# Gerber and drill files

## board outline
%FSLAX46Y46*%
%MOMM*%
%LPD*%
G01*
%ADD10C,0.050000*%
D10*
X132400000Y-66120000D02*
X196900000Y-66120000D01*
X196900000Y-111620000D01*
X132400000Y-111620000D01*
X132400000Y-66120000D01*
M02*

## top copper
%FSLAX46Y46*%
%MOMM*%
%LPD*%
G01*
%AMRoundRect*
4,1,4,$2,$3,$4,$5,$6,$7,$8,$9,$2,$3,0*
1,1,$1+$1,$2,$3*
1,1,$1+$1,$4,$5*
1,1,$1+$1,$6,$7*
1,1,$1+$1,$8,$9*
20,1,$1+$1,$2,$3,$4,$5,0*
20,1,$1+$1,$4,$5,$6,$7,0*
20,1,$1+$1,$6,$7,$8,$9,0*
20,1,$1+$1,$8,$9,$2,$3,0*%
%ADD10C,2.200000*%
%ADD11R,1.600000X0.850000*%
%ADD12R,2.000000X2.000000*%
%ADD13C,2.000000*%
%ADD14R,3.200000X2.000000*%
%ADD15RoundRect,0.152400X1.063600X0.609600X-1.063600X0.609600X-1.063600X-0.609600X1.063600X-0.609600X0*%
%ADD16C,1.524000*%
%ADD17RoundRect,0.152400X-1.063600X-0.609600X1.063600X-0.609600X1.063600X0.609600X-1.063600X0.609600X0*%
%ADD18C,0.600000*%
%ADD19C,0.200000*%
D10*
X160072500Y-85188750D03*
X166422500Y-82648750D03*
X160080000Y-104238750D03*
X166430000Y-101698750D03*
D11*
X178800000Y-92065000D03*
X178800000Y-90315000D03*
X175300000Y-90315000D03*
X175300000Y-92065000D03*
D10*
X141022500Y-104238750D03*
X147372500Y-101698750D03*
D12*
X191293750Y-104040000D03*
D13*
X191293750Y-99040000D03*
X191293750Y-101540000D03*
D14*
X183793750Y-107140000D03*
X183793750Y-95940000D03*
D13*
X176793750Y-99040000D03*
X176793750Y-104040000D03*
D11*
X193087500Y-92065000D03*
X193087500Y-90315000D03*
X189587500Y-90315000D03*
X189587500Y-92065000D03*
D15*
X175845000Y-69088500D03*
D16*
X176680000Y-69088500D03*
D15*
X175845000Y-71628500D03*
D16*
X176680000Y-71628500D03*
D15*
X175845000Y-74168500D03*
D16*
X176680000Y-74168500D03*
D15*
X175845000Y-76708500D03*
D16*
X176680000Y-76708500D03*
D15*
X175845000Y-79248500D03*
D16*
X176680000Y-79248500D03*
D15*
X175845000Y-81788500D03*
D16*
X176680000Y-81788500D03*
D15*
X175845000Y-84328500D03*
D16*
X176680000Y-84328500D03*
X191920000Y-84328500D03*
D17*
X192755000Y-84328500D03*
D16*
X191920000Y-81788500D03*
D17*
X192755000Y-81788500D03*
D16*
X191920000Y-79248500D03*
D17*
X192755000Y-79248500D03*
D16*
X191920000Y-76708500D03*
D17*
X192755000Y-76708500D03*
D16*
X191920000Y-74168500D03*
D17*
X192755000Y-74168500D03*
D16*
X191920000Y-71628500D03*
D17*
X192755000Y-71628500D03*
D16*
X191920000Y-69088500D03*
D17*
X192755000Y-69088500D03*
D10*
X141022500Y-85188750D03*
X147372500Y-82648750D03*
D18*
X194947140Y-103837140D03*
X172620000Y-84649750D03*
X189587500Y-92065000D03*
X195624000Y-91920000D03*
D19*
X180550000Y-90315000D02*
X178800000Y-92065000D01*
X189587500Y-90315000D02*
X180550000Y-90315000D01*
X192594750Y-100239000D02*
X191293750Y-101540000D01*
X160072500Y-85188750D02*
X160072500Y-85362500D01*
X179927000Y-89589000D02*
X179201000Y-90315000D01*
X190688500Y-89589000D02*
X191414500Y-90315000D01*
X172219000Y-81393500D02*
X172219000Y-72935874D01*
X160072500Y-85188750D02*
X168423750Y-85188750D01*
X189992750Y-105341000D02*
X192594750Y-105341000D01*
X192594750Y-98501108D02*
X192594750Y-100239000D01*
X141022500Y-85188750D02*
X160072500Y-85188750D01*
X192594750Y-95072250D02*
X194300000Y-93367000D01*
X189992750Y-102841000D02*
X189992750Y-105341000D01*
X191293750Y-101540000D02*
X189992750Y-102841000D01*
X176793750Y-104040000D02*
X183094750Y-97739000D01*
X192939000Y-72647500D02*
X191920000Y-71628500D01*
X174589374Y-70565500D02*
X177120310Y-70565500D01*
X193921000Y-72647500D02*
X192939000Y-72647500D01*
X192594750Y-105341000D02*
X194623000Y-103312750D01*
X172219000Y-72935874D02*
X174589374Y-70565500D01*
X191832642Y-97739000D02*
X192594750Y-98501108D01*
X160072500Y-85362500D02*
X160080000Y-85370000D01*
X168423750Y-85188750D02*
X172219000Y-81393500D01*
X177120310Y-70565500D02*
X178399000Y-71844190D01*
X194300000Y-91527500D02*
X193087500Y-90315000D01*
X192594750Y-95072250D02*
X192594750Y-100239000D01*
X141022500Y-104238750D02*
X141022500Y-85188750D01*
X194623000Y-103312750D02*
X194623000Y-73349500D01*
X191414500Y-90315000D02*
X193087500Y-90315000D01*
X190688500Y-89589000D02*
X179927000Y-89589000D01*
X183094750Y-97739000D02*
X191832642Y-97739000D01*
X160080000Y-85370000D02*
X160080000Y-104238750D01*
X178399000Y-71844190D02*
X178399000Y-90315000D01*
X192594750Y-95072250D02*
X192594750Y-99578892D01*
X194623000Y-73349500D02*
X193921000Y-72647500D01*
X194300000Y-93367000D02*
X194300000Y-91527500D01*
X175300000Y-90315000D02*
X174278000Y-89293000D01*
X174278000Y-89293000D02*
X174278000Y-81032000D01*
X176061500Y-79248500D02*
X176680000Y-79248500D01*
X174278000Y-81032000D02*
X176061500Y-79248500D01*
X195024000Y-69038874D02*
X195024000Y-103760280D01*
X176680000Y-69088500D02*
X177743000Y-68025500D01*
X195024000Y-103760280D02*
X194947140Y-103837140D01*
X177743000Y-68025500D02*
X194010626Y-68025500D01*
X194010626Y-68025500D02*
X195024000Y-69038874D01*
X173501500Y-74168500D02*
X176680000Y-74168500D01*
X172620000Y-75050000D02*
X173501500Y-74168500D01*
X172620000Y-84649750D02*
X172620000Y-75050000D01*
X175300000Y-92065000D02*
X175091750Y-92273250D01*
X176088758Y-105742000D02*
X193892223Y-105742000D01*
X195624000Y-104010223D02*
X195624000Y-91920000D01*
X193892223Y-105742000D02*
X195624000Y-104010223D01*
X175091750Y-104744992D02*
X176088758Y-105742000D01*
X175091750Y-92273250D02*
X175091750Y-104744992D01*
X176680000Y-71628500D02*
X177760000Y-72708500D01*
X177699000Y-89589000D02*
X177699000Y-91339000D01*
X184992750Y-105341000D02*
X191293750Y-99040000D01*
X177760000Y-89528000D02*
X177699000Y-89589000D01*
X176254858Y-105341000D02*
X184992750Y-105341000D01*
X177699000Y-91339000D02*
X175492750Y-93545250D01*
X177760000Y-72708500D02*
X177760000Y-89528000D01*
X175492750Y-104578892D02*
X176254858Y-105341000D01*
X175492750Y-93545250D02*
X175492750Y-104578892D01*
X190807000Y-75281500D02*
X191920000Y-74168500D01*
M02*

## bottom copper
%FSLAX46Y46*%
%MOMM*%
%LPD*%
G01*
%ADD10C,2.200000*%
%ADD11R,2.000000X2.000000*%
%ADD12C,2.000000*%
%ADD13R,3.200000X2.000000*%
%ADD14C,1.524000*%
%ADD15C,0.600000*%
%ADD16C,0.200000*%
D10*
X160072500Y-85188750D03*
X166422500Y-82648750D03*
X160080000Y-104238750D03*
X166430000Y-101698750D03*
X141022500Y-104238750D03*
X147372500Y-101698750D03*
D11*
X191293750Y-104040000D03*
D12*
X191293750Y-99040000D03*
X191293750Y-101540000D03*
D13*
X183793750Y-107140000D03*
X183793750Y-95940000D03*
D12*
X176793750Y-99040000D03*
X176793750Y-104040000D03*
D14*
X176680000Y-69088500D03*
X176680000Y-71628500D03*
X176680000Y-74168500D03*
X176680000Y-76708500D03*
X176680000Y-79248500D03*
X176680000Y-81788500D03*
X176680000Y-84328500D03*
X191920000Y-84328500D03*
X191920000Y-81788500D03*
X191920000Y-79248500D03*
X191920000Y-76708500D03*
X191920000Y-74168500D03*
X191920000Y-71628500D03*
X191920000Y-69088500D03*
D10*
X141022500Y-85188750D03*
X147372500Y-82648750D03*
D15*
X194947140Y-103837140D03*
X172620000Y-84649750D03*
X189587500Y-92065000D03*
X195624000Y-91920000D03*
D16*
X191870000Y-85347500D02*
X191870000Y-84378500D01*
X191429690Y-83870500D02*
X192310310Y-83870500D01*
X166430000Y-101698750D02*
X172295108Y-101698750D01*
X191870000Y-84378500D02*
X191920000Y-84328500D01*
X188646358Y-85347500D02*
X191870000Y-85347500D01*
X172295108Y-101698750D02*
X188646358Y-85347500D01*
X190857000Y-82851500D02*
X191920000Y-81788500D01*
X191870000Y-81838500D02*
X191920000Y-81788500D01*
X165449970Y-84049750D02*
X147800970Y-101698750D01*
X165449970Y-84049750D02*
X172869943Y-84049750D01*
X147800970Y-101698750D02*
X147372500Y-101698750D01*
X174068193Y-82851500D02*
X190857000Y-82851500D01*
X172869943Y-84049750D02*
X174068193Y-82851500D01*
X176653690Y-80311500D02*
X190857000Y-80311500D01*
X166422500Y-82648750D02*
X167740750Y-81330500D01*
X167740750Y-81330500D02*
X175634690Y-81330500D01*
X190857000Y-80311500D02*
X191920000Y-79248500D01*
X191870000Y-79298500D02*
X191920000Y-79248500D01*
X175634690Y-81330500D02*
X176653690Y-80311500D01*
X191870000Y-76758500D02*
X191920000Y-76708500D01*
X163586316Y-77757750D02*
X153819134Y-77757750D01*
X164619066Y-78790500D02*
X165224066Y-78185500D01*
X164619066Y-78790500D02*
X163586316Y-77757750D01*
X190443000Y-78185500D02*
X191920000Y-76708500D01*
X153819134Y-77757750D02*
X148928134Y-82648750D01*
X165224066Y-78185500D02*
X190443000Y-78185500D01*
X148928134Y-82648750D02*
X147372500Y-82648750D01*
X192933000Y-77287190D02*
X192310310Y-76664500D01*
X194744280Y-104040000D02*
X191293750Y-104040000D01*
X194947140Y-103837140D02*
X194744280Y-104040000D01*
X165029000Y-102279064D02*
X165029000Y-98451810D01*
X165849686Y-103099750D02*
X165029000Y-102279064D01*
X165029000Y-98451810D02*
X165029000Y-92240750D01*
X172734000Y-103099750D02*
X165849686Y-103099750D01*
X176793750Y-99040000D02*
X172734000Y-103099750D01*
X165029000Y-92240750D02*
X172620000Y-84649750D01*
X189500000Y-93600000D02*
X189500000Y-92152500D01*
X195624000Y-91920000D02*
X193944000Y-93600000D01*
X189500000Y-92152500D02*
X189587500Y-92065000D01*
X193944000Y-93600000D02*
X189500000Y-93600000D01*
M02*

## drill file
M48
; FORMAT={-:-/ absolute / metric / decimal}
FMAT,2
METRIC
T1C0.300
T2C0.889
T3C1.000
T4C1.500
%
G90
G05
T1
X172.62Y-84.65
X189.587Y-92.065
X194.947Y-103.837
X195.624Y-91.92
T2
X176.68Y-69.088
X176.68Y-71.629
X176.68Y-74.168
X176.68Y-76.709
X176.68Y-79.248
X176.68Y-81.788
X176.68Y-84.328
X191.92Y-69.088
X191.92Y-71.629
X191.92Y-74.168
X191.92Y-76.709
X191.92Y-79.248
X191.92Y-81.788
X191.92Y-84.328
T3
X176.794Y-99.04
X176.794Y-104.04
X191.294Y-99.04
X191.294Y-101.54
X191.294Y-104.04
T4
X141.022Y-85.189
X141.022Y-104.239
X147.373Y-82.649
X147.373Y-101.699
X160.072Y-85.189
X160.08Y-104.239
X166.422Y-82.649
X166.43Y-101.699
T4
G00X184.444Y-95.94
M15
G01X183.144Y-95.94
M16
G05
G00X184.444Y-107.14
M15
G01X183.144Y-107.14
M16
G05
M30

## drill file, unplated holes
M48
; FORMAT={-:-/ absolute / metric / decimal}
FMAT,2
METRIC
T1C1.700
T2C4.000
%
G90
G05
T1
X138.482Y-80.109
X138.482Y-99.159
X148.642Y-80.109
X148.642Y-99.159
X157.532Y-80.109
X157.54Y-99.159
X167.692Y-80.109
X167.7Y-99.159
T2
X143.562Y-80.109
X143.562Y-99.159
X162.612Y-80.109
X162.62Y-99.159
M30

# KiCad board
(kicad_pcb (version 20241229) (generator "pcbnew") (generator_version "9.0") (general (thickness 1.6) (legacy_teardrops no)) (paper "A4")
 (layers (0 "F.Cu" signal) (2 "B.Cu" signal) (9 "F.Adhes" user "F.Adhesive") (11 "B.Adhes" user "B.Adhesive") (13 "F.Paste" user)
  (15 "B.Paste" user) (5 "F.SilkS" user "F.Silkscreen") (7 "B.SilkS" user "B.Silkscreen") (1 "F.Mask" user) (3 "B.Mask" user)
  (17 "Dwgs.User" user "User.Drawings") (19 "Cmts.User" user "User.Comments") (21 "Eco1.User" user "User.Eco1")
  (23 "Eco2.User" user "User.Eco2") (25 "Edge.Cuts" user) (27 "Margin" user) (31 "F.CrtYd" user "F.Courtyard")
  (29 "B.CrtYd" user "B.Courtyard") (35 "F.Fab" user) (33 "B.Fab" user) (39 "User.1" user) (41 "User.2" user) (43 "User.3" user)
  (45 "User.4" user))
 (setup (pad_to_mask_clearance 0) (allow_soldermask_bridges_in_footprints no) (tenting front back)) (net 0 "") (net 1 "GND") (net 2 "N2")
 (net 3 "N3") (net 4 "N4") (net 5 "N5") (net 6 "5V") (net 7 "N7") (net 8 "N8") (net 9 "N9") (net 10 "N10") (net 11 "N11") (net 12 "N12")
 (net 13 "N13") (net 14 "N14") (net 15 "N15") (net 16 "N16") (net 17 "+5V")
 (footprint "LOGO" (layer "F.Cu") (at 188.806519 109.90525 180)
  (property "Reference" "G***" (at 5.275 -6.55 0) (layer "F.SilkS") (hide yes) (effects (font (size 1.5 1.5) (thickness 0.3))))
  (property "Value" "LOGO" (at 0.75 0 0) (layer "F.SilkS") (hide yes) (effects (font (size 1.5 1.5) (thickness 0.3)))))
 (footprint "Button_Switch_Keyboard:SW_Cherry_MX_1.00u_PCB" (layer "F.Cu") (at 160.0725 85.18875 180)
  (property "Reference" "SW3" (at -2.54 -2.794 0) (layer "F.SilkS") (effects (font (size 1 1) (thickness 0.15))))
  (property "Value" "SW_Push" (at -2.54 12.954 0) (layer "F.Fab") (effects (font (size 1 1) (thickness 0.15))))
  (pad "" np_thru_hole circle (at -7.62 5.08 180) (size 1.7 1.7) (drill 1.7) (layers "*.Cu" "*.Mask"))
  (pad "" np_thru_hole circle (at -2.54 5.08 180) (size 4 4) (drill 4) (layers "*.Cu" "*.Mask"))
  (pad "" np_thru_hole circle (at 2.54 5.08 180) (size 1.7 1.7) (drill 1.7) (layers "*.Cu" "*.Mask"))
  (pad "1" thru_hole circle (at 0 0 180) (size 2.2 2.2) (drill 1.5) (layers "*.Cu" "*.Mask") (remove_unused_layers no) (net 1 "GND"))
  (pad "2" thru_hole circle (at -6.35 2.54 180) (size 2.2 2.2) (drill 1.5) (layers "*.Cu" "*.Mask") (remove_unused_layers no) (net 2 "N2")))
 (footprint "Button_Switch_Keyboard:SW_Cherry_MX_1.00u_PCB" (layer "F.Cu") (at 160.08 104.23875 180)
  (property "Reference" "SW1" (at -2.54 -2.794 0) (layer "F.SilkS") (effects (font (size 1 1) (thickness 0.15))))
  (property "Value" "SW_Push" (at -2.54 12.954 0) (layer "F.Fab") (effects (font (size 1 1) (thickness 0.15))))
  (pad "" np_thru_hole circle (at -7.62 5.08 180) (size 1.7 1.7) (drill 1.7) (layers "*.Cu" "*.Mask"))
  (pad "" np_thru_hole circle (at -2.54 5.08 180) (size 4 4) (drill 4) (layers "*.Cu" "*.Mask"))
  (pad "" np_thru_hole circle (at 2.54 5.08 180) (size 1.7 1.7) (drill 1.7) (layers "*.Cu" "*.Mask"))
  (pad "1" thru_hole circle (at 0 0 180) (size 2.2 2.2) (drill 1.5) (layers "*.Cu" "*.Mask") (remove_unused_layers no) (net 1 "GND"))
  (pad "2" thru_hole circle (at -6.35 2.54 180) (size 2.2 2.2) (drill 1.5) (layers "*.Cu" "*.Mask") (remove_unused_layers no) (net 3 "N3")))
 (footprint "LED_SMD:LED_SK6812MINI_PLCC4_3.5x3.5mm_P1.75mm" (layer "F.Cu") (at 177.05 91.19 180)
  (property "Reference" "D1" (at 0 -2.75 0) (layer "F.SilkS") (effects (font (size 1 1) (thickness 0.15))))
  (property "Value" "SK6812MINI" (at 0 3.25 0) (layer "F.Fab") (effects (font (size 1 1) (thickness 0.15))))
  (pad "1" smd rect (at -1.75 -0.875 180) (size 1.6 0.85) (layers "F.Cu" "F.Mask" "F.Paste") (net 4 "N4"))
  (pad "2" smd rect (at -1.75 0.875 180) (size 1.6 0.85) (layers "F.Cu" "F.Mask" "F.Paste") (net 1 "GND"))
  (pad "3" smd rect (at 1.75 0.875 180) (size 1.6 0.85) (layers "F.Cu" "F.Mask" "F.Paste") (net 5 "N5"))
  (pad "4" smd rect (at 1.75 -0.875 180) (size 1.6 0.85) (layers "F.Cu" "F.Mask" "F.Paste") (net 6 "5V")))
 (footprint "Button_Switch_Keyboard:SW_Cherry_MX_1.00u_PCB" (layer "F.Cu") (at 141.0225 104.23875 180)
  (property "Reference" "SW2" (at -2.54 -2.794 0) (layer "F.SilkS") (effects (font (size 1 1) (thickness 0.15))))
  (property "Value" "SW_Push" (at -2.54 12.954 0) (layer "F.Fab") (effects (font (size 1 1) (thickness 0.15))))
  (pad "" np_thru_hole circle (at -7.62 5.08 180) (size 1.7 1.7) (drill 1.7) (layers "*.Cu" "*.Mask"))
  (pad "" np_thru_hole circle (at -2.54 5.08 180) (size 4 4) (drill 4) (layers "*.Cu" "*.Mask"))
  (pad "" np_thru_hole circle (at 2.54 5.08 180) (size 1.7 1.7) (drill 1.7) (layers "*.Cu" "*.Mask"))
  (pad "1" thru_hole circle (at 0 0 180) (size 2.2 2.2) (drill 1.5) (layers "*.Cu" "*.Mask") (remove_unused_layers no) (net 1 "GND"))
  (pad "2" thru_hole circle (at -6.35 2.54 180) (size 2.2 2.2) (drill 1.5) (layers "*.Cu" "*.Mask") (remove_unused_layers no) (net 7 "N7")))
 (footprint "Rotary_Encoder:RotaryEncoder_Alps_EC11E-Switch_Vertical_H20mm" (layer "F.Cu") (at 191.29375 104.04 180)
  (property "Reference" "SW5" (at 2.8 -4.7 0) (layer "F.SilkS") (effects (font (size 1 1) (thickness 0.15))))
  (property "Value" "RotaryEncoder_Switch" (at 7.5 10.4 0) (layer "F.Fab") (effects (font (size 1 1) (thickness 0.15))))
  (pad "A" thru_hole rect (at 0 0 180) (size 2 2) (drill 1) (layers "*.Cu" "*.Mask") (remove_unused_layers no) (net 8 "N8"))
  (pad "B" thru_hole circle (at 0 5 180) (size 2 2) (drill 1) (layers "*.Cu" "*.Mask") (remove_unused_layers no) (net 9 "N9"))
  (pad "C" thru_hole circle (at 0 2.5 180) (size 2 2) (drill 1) (layers "*.Cu" "*.Mask") (remove_unused_layers no) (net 1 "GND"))
  (pad "MP" thru_hole rect (at 7.5 -3.1 180) (size 3.2 2) (drill oval 2.8 1.5) (layers "*.Cu" "*.Mask") (remove_unused_layers no))
  (pad "MP" thru_hole rect (at 7.5 8.1 180) (size 3.2 2) (drill oval 2.8 1.5) (layers "*.Cu" "*.Mask") (remove_unused_layers no))
  (pad "S1" thru_hole circle (at 14.5 5 180) (size 2 2) (drill 1) (layers "*.Cu" "*.Mask") (remove_unused_layers no) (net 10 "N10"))
  (pad "S2" thru_hole circle (at 14.5 0 180) (size 2 2) (drill 1) (layers "*.Cu" "*.Mask") (remove_unused_layers no) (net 1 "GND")))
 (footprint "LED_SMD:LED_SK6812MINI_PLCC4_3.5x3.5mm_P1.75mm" (layer "F.Cu") (at 191.3375 91.19 180)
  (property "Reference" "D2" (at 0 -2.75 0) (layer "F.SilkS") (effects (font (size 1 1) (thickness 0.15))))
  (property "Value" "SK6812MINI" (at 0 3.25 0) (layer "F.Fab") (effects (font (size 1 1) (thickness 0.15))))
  (pad "1" smd rect (at -1.75 -0.875 180) (size 1.6 0.85) (layers "F.Cu" "F.Mask" "F.Paste") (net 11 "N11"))
  (pad "2" smd rect (at -1.75 0.875 180) (size 1.6 0.85) (layers "F.Cu" "F.Mask" "F.Paste") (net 1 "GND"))
  (pad "3" smd rect (at 1.75 0.875 180) (size 1.6 0.85) (layers "F.Cu" "F.Mask" "F.Paste") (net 4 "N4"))
  (pad "4" smd rect (at 1.75 -0.875 180) (size 1.6 0.85) (layers "F.Cu" "F.Mask" "F.Paste") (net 6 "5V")))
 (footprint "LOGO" (layer "F.Cu") (at 139.886519 110.04525 180)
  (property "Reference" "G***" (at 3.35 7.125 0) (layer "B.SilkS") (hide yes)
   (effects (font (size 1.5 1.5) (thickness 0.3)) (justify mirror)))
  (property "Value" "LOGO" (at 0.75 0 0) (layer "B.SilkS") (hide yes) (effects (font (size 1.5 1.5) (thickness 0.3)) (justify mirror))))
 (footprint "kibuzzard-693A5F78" (layer "F.Cu") (at 153.025 69.69)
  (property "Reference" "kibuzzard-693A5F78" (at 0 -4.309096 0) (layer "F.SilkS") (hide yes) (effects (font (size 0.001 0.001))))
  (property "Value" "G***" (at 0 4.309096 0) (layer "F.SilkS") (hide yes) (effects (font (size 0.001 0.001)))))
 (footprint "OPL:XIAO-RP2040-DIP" (layer "F.Cu") (at 184.3 76.7085)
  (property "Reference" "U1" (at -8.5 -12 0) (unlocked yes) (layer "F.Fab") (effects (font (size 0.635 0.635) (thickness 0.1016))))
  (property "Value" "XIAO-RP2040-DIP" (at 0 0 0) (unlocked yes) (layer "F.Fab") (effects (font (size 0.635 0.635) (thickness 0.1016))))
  (pad "1" smd roundrect (at -8.455 -7.62 180) (size 2.432 1.524) (layers "F.Cu" "F.Mask") (roundrect_rratio 0.1) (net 8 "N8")
   (thermal_bridge_angle 45))
  (pad "1" thru_hole circle (at -7.62 -7.62 180) (size 1.524 1.524) (drill 0.889) (layers "*.Cu" "*.Mask") (remove_unused_layers no)
   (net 8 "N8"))
  (pad "2" smd roundrect (at -8.455 -5.08 180) (size 2.432 1.524) (layers "F.Cu" "F.Mask") (roundrect_rratio 0.1) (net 9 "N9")
   (thermal_bridge_angle 45))
  (pad "2" thru_hole circle (at -7.62 -5.08 180) (size 1.524 1.524) (drill 0.889) (layers "*.Cu" "*.Mask") (remove_unused_layers no)
   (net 9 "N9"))
  (pad "3" smd roundrect (at -8.455 -2.54 180) (size 2.432 1.524) (layers "F.Cu" "F.Mask") (roundrect_rratio 0.1) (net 10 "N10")
   (thermal_bridge_angle 45))
  (pad "3" thru_hole circle (at -7.62 -2.54 180) (size 1.524 1.524) (drill 0.889) (layers "*.Cu" "*.Mask") (remove_unused_layers no)
   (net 10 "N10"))
  (pad "4" smd roundrect (at -8.455 0 180) (size 2.432 1.524) (layers "F.Cu" "F.Mask") (roundrect_rratio 0.1) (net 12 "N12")
   (thermal_bridge_angle 45))
  (pad "4" thru_hole circle (at -7.62 0 180) (size 1.524 1.524) (drill 0.889) (layers "*.Cu" "*.Mask") (remove_unused_layers no)
   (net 12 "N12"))
  (pad "5" smd roundrect (at -8.455 2.54 180) (size 2.432 1.524) (layers "F.Cu" "F.Mask") (roundrect_rratio 0.1) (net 5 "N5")
   (thermal_bridge_angle 45))
  (pad "5" thru_hole circle (at -7.62 2.54 180) (size 1.524 1.524) (drill 0.889) (layers "*.Cu" "*.Mask") (remove_unused_layers no)
   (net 5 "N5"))
  (pad "6" smd roundrect (at -8.455 5.08 180) (size 2.432 1.524) (layers "F.Cu" "F.Mask") (roundrect_rratio 0.1) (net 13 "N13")
   (thermal_bridge_angle 45))
  (pad "6" thru_hole circle (at -7.62 5.08 180) (size 1.524 1.524) (drill 0.889) (layers "*.Cu" "*.Mask") (remove_unused_layers no)
   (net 13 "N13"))
  (pad "7" smd roundrect (at -8.455 7.62 180) (size 2.432 1.524) (layers "F.Cu" "F.Mask") (roundrect_rratio 0.1) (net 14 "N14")
   (thermal_bridge_angle 45))
  (pad "7" thru_hole circle (at -7.62 7.62 180) (size 1.524 1.524) (drill 0.889) (layers "*.Cu" "*.Mask") (remove_unused_layers no)
   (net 14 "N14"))
  (pad "8" thru_hole circle (at 7.62 7.62) (size 1.524 1.524) (drill 0.889) (layers "*.Cu" "*.Mask") (remove_unused_layers no) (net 3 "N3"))
  (pad "8" smd roundrect (at 8.455 7.62) (size 2.432 1.524) (layers "F.Cu" "F.Mask") (roundrect_rratio 0.1) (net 3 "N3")
   (thermal_bridge_angle 45))
  (pad "9" thru_hole circle (at 7.62 5.08) (size 1.524 1.524) (drill 0.889) (layers "*.Cu" "*.Mask") (remove_unused_layers no) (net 7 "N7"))
  (pad "9" smd roundrect (at 8.455 5.08) (size 2.432 1.524) (layers "F.Cu" "F.Mask") (roundrect_rratio 0.1) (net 7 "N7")
   (thermal_bridge_angle 45))
  (pad "10" thru_hole circle (at 7.62 2.54) (size 1.524 1.524) (drill 0.889) (layers "*.Cu" "*.Mask") (remove_unused_layers no) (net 2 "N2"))
  (pad "10" smd roundrect (at 8.455 2.54) (size 2.432 1.524) (layers "F.Cu" "F.Mask") (roundrect_rratio 0.1) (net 2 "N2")
   (thermal_bridge_angle 45))
  (pad "11" thru_hole circle (at 7.62 0) (size 1.524 1.524) (drill 0.889) (layers "*.Cu" "*.Mask") (remove_unused_layers no) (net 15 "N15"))
  (pad "11" smd roundrect (at 8.455 0) (size 2.432 1.524) (layers "F.Cu" "F.Mask") (roundrect_rratio 0.1) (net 15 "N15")
   (thermal_bridge_angle 45))
  (pad "12" thru_hole circle (at 7.62 -2.54) (size 1.524 1.524) (drill 0.889) (layers "*.Cu" "*.Mask") (remove_unused_layers no)
   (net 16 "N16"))
  (pad "12" smd roundrect (at 8.455 -2.54) (size 2.432 1.524) (layers "F.Cu" "F.Mask") (roundrect_rratio 0.1) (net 16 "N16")
   (thermal_bridge_angle 45))
  (pad "13" thru_hole circle (at 7.62 -5.08) (size 1.524 1.524) (drill 0.889) (layers "*.Cu" "*.Mask") (remove_unused_layers no)
   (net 1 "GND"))
  (pad "13" smd roundrect (at 8.455 -5.08) (size 2.432 1.524) (layers "F.Cu" "F.Mask") (roundrect_rratio 0.1) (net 1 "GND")
   (thermal_bridge_angle 45))
  (pad "14" thru_hole circle (at 7.62 -7.62) (size 1.524 1.524) (drill 0.889) (layers "*.Cu" "*.Mask") (remove_unused_layers no)
   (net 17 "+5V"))
  (pad "14" smd roundrect (at 8.455 -7.62) (size 2.432 1.524) (layers "F.Cu" "F.Mask") (roundrect_rratio 0.1) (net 17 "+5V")
   (thermal_bridge_angle 45)))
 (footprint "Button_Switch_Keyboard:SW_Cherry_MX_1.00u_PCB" (layer "F.Cu") (at 141.0225 85.18875 180)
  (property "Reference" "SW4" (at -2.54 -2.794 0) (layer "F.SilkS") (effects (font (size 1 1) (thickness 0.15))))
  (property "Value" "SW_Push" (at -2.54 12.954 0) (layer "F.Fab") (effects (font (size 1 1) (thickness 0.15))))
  (pad "" np_thru_hole circle (at -7.62 5.08 180) (size 1.7 1.7) (drill 1.7) (layers "*.Cu" "*.Mask"))
  (pad "" np_thru_hole circle (at -2.54 5.08 180) (size 4 4) (drill 4) (layers "*.Cu" "*.Mask"))
  (pad "" np_thru_hole circle (at 2.54 5.08 180) (size 1.7 1.7) (drill 1.7) (layers "*.Cu" "*.Mask"))
  (pad "1" thru_hole circle (at 0 0 180) (size 2.2 2.2) (drill 1.5) (layers "*.Cu" "*.Mask") (remove_unused_layers no) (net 1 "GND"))
  (pad "2" thru_hole circle (at -6.35 2.54 180) (size 2.2 2.2) (drill 1.5) (layers "*.Cu" "*.Mask") (remove_unused_layers no) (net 15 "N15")))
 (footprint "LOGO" (layer "B.Cu") (at 141.654429 68.782568)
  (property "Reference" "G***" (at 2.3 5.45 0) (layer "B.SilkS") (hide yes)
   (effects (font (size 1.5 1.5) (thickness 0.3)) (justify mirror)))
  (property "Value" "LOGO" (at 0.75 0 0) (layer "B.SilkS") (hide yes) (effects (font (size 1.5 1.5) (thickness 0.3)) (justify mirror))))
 (gr_rect (start 132.4 66.12) (end 196.9 111.62) (stroke (width 0.05) (type solid)) (fill no) (layer "Edge.Cuts"))
 (segment (start 180.55 90.315) (end 178.8 92.065) (width 0.2) (layer "F.Cu") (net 4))
 (segment (start 189.5875 90.315) (end 180.55 90.315) (width 0.2) (layer "F.Cu") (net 4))
 (segment (start 192.59475 100.239) (end 191.29375 101.54) (width 0.2) (layer "F.Cu") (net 1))
 (segment (start 160.0725 85.18875) (end 160.0725 85.3625) (width 0.2) (layer "F.Cu") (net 1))
 (segment (start 179.927 89.589) (end 179.201 90.315) (width 0.2) (layer "F.Cu") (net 1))
 (segment (start 190.6885 89.589) (end 191.4145 90.315) (width 0.2) (layer "F.Cu") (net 1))
 (segment (start 172.219 81.3935) (end 172.219 72.935874) (width 0.2) (layer "F.Cu") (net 1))
 (segment (start 160.0725 85.18875) (end 168.42375 85.18875) (width 0.2) (layer "F.Cu") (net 1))
 (segment (start 189.99275 105.341) (end 192.59475 105.341) (width 0.2) (layer "F.Cu") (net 1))
 (segment (start 192.59475 98.501108) (end 192.59475 100.239) (width 0.2) (layer "F.Cu") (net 1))
 (segment (start 141.0225 85.18875) (end 160.0725 85.18875) (width 0.2) (layer "F.Cu") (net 1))
 (segment (start 192.59475 95.07225) (end 194.3 93.367) (width 0.2) (layer "F.Cu") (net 1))
 (segment (start 189.99275 102.841) (end 189.99275 105.341) (width 0.2) (layer "F.Cu") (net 1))
 (segment (start 191.29375 101.54) (end 189.99275 102.841) (width 0.2) (layer "F.Cu") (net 1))
 (segment (start 176.79375 104.04) (end 183.09475 97.739) (width 0.2) (layer "F.Cu") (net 1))
 (segment (start 192.939 72.6475) (end 191.92 71.6285) (width 0.2) (layer "F.Cu") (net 1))
 (segment (start 174.589374 70.5655) (end 177.12031 70.5655) (width 0.2) (layer "F.Cu") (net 1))
 (segment (start 193.921 72.6475) (end 192.939 72.6475) (width 0.2) (layer "F.Cu") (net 1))
 (segment (start 192.59475 105.341) (end 194.623 103.31275) (width 0.2) (layer "F.Cu") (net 1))
 (segment (start 172.219 72.935874) (end 174.589374 70.5655) (width 0.2) (layer "F.Cu") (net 1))
 (segment (start 191.832642 97.739) (end 192.59475 98.501108) (width 0.2) (layer "F.Cu") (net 1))
 (segment (start 160.0725 85.3625) (end 160.08 85.37) (width 0.2) (layer "F.Cu") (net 1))
 (segment (start 168.42375 85.18875) (end 172.219 81.3935) (width 0.2) (layer "F.Cu") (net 1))
 (segment (start 177.12031 70.5655) (end 178.399 71.84419) (width 0.2) (layer "F.Cu") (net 1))
 (segment (start 194.3 91.5275) (end 193.0875 90.315) (width 0.2) (layer "F.Cu") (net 1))
 (segment (start 192.59475 95.07225) (end 192.59475 100.239) (width 0.2) (layer "F.Cu") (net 1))
 (segment (start 141.0225 104.23875) (end 141.0225 85.18875) (width 0.2) (layer "F.Cu") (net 1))
 (segment (start 194.623 103.31275) (end 194.623 73.3495) (width 0.2) (layer "F.Cu") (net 1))
 (segment (start 191.4145 90.315) (end 193.0875 90.315) (width 0.2) (layer "F.Cu") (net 1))
 (segment (start 190.6885 89.589) (end 179.927 89.589) (width 0.2) (layer "F.Cu") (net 1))
 (segment (start 183.09475 97.739) (end 191.832642 97.739) (width 0.2) (layer "F.Cu") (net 1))
 (segment (start 160.08 85.37) (end 160.08 104.23875) (width 0.2) (layer "F.Cu") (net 1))
 (segment (start 178.399 71.84419) (end 178.399 90.315) (width 0.2) (layer "F.Cu") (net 1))
 (segment (start 192.59475 95.07225) (end 192.59475 99.578892) (width 0.2) (layer "F.Cu") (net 1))
 (segment (start 194.623 73.3495) (end 193.921 72.6475) (width 0.2) (layer "F.Cu") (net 1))
 (segment (start 194.3 93.367) (end 194.3 91.5275) (width 0.2) (layer "F.Cu") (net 1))
 (segment (start 175.3 90.315) (end 174.278 89.293) (width 0.2) (layer "F.Cu") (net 5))
 (segment (start 174.278 89.293) (end 174.278 81.032) (width 0.2) (layer "F.Cu") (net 5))
 (segment (start 176.0615 79.2485) (end 176.68 79.2485) (width 0.2) (layer "F.Cu") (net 5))
 (segment (start 174.278 81.032) (end 176.0615 79.2485) (width 0.2) (layer "F.Cu") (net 5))
 (segment (start 191.87 85.3475) (end 191.87 84.3785) (width 0.2) (layer "B.Cu") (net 3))
 (segment (start 191.42969 83.8705) (end 192.31031 83.8705) (width 0.2) (layer "B.Cu") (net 3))
 (segment (start 166.43 101.69875) (end 172.295108 101.69875) (width 0.2) (layer "B.Cu") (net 3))
 (segment (start 191.87 84.3785) (end 191.92 84.3285) (width 0.2) (layer "B.Cu") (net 3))
 (segment (start 188.646358 85.3475) (end 191.87 85.3475) (width 0.2) (layer "B.Cu") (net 3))
 (segment (start 172.295108 101.69875) (end 188.646358 85.3475) (width 0.2) (layer "B.Cu") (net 3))
 (segment (start 190.857 82.8515) (end 191.92 81.7885) (width 0.2) (layer "B.Cu") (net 7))
 (segment (start 191.87 81.8385) (end 191.92 81.7885) (width 0.2) (layer "B.Cu") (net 7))
 (segment (start 165.44997 84.04975) (end 147.80097 101.69875) (width 0.2) (layer "B.Cu") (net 7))
 (segment (start 165.44997 84.04975) (end 172.869943 84.04975) (width 0.2) (layer "B.Cu") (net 7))
 (segment (start 147.80097 101.69875) (end 147.3725 101.69875) (width 0.2) (layer "B.Cu") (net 7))
 (segment (start 174.068193 82.8515) (end 190.857 82.8515) (width 0.2) (layer "B.Cu") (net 7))
 (segment (start 172.869943 84.04975) (end 174.068193 82.8515) (width 0.2) (layer "B.Cu") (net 7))
 (segment (start 176.65369 80.3115) (end 190.857 80.3115) (width 0.2) (layer "B.Cu") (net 2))
 (segment (start 166.4225 82.64875) (end 167.74075 81.3305) (width 0.2) (layer "B.Cu") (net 2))
 (segment (start 167.74075 81.3305) (end 175.63469 81.3305) (width 0.2) (layer "B.Cu") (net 2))
 (segment (start 190.857 80.3115) (end 191.92 79.2485) (width 0.2) (layer "B.Cu") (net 2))
 (segment (start 191.87 79.2985) (end 191.92 79.2485) (width 0.2) (layer "B.Cu") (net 2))
 (segment (start 175.63469 81.3305) (end 176.65369 80.3115) (width 0.2) (layer "B.Cu") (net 2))
 (segment (start 191.87 76.7585) (end 191.92 76.7085) (width 0.2) (layer "B.Cu") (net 15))
 (segment (start 163.586316 77.75775) (end 153.819134 77.75775) (width 0.2) (layer "B.Cu") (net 15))
 (segment (start 164.619066 78.7905) (end 165.224066 78.1855) (width 0.2) (layer "B.Cu") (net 15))
 (segment (start 164.619066 78.7905) (end 163.586316 77.75775) (width 0.2) (layer "B.Cu") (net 15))
 (segment (start 190.443 78.1855) (end 191.92 76.7085) (width 0.2) (layer "B.Cu") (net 15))
 (segment (start 153.819134 77.75775) (end 148.928134 82.64875) (width 0.2) (layer "B.Cu") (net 15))
 (segment (start 165.224066 78.1855) (end 190.443 78.1855) (width 0.2) (layer "B.Cu") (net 15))
 (segment (start 148.928134 82.64875) (end 147.3725 82.64875) (width 0.2) (layer "B.Cu") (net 15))
 (segment (start 192.933 77.28719) (end 192.31031 76.6645) (width 0.2) (layer "B.Cu") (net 15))
 (segment (start 195.024 69.038874) (end 195.024 103.76028) (width 0.2) (layer "F.Cu") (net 8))
 (segment (start 176.68 69.0885) (end 177.743 68.0255) (width 0.2) (layer "F.Cu") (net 8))
 (segment (start 195.024 103.76028) (end 194.94714 103.83714) (width 0.2) (layer "F.Cu") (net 8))
 (segment (start 177.743 68.0255) (end 194.010626 68.0255) (width 0.2) (layer "F.Cu") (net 8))
 (segment (start 194.010626 68.0255) (end 195.024 69.038874) (width 0.2) (layer "F.Cu") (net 8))
 (via (at 194.94714 103.83714) (size 0.6) (drill 0.3) (layers "F.Cu" "B.Cu") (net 8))
 (segment (start 194.74428 104.04) (end 191.29375 104.04) (width 0.2) (layer "B.Cu") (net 8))
 (segment (start 194.94714 103.83714) (end 194.74428 104.04) (width 0.2) (layer "B.Cu") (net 8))
 (segment (start 173.5015 74.1685) (end 176.68 74.1685) (width 0.2) (layer "F.Cu") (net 10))
 (segment (start 172.62 75.05) (end 173.5015 74.1685) (width 0.2) (layer "F.Cu") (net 10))
 (segment (start 172.62 84.64975) (end 172.62 75.05) (width 0.2) (layer "F.Cu") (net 10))
 (via (at 172.62 84.64975) (size 0.6) (drill 0.3) (layers "F.Cu" "B.Cu") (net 10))
 (segment (start 165.029 102.279064) (end 165.029 98.45181) (width 0.2) (layer "B.Cu") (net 10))
 (segment (start 165.849686 103.09975) (end 165.029 102.279064) (width 0.2) (layer "B.Cu") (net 10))
 (segment (start 165.029 98.45181) (end 165.029 92.24075) (width 0.2) (layer "B.Cu") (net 10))
 (segment (start 172.734 103.09975) (end 165.849686 103.09975) (width 0.2) (layer "B.Cu") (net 10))
 (segment (start 176.79375 99.04) (end 172.734 103.09975) (width 0.2) (layer "B.Cu") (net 10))
 (segment (start 165.029 92.24075) (end 172.62 84.64975) (width 0.2) (layer "B.Cu") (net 10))
 (segment (start 175.3 92.065) (end 175.09175 92.27325) (width 0.2) (layer "F.Cu") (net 6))
 (segment (start 176.088758 105.742) (end 193.892223 105.742) (width 0.2) (layer "F.Cu") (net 6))
 (segment (start 195.624 104.010223) (end 195.624 91.92) (width 0.2) (layer "F.Cu") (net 6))
 (segment (start 193.892223 105.742) (end 195.624 104.010223) (width 0.2) (layer "F.Cu") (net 6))
 (segment (start 175.09175 104.744992) (end 176.088758 105.742) (width 0.2) (layer "F.Cu") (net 6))
 (segment (start 175.09175 92.27325) (end 175.09175 104.744992) (width 0.2) (layer "F.Cu") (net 6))
 (via (at 189.5875 92.065) (size 0.6) (drill 0.3) (layers "F.Cu" "B.Cu") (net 6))
 (via (at 195.624 91.92) (size 0.6) (drill 0.3) (layers "F.Cu" "B.Cu") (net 6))
 (segment (start 189.5 93.6) (end 189.5 92.1525) (width 0.2) (layer "B.Cu") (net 6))
 (segment (start 195.624 91.92) (end 193.944 93.6) (width 0.2) (layer "B.Cu") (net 6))
 (segment (start 189.5 92.1525) (end 189.5875 92.065) (width 0.2) (layer "B.Cu") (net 6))
 (segment (start 193.944 93.6) (end 189.5 93.6) (width 0.2) (layer "B.Cu") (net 6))
 (segment (start 176.68 71.6285) (end 177.76 72.7085) (width 0.2) (layer "F.Cu") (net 9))
 (segment (start 177.699 89.589) (end 177.699 91.339) (width 0.2) (layer "F.Cu") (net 9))
 (segment (start 184.99275 105.341) (end 191.29375 99.04) (width 0.2) (layer "F.Cu") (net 9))
 (segment (start 177.76 89.528) (end 177.699 89.589) (width 0.2) (layer "F.Cu") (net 9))
 (segment (start 176.254858 105.341) (end 184.99275 105.341) (width 0.2) (layer "F.Cu") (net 9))
 (segment (start 177.699 91.339) (end 175.49275 93.54525) (width 0.2) (layer "F.Cu") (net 9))
 (segment (start 177.76 72.7085) (end 177.76 89.528) (width 0.2) (layer "F.Cu") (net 9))
 (segment (start 175.49275 104.578892) (end 176.254858 105.341) (width 0.2) (layer "F.Cu") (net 9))
 (segment (start 175.49275 93.54525) (end 175.49275 104.578892) (width 0.2) (layer "F.Cu") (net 9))
 (segment (start 190.807 75.2815) (end 191.92 74.1685) (width 0.2) (layer "F.Cu") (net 16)))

